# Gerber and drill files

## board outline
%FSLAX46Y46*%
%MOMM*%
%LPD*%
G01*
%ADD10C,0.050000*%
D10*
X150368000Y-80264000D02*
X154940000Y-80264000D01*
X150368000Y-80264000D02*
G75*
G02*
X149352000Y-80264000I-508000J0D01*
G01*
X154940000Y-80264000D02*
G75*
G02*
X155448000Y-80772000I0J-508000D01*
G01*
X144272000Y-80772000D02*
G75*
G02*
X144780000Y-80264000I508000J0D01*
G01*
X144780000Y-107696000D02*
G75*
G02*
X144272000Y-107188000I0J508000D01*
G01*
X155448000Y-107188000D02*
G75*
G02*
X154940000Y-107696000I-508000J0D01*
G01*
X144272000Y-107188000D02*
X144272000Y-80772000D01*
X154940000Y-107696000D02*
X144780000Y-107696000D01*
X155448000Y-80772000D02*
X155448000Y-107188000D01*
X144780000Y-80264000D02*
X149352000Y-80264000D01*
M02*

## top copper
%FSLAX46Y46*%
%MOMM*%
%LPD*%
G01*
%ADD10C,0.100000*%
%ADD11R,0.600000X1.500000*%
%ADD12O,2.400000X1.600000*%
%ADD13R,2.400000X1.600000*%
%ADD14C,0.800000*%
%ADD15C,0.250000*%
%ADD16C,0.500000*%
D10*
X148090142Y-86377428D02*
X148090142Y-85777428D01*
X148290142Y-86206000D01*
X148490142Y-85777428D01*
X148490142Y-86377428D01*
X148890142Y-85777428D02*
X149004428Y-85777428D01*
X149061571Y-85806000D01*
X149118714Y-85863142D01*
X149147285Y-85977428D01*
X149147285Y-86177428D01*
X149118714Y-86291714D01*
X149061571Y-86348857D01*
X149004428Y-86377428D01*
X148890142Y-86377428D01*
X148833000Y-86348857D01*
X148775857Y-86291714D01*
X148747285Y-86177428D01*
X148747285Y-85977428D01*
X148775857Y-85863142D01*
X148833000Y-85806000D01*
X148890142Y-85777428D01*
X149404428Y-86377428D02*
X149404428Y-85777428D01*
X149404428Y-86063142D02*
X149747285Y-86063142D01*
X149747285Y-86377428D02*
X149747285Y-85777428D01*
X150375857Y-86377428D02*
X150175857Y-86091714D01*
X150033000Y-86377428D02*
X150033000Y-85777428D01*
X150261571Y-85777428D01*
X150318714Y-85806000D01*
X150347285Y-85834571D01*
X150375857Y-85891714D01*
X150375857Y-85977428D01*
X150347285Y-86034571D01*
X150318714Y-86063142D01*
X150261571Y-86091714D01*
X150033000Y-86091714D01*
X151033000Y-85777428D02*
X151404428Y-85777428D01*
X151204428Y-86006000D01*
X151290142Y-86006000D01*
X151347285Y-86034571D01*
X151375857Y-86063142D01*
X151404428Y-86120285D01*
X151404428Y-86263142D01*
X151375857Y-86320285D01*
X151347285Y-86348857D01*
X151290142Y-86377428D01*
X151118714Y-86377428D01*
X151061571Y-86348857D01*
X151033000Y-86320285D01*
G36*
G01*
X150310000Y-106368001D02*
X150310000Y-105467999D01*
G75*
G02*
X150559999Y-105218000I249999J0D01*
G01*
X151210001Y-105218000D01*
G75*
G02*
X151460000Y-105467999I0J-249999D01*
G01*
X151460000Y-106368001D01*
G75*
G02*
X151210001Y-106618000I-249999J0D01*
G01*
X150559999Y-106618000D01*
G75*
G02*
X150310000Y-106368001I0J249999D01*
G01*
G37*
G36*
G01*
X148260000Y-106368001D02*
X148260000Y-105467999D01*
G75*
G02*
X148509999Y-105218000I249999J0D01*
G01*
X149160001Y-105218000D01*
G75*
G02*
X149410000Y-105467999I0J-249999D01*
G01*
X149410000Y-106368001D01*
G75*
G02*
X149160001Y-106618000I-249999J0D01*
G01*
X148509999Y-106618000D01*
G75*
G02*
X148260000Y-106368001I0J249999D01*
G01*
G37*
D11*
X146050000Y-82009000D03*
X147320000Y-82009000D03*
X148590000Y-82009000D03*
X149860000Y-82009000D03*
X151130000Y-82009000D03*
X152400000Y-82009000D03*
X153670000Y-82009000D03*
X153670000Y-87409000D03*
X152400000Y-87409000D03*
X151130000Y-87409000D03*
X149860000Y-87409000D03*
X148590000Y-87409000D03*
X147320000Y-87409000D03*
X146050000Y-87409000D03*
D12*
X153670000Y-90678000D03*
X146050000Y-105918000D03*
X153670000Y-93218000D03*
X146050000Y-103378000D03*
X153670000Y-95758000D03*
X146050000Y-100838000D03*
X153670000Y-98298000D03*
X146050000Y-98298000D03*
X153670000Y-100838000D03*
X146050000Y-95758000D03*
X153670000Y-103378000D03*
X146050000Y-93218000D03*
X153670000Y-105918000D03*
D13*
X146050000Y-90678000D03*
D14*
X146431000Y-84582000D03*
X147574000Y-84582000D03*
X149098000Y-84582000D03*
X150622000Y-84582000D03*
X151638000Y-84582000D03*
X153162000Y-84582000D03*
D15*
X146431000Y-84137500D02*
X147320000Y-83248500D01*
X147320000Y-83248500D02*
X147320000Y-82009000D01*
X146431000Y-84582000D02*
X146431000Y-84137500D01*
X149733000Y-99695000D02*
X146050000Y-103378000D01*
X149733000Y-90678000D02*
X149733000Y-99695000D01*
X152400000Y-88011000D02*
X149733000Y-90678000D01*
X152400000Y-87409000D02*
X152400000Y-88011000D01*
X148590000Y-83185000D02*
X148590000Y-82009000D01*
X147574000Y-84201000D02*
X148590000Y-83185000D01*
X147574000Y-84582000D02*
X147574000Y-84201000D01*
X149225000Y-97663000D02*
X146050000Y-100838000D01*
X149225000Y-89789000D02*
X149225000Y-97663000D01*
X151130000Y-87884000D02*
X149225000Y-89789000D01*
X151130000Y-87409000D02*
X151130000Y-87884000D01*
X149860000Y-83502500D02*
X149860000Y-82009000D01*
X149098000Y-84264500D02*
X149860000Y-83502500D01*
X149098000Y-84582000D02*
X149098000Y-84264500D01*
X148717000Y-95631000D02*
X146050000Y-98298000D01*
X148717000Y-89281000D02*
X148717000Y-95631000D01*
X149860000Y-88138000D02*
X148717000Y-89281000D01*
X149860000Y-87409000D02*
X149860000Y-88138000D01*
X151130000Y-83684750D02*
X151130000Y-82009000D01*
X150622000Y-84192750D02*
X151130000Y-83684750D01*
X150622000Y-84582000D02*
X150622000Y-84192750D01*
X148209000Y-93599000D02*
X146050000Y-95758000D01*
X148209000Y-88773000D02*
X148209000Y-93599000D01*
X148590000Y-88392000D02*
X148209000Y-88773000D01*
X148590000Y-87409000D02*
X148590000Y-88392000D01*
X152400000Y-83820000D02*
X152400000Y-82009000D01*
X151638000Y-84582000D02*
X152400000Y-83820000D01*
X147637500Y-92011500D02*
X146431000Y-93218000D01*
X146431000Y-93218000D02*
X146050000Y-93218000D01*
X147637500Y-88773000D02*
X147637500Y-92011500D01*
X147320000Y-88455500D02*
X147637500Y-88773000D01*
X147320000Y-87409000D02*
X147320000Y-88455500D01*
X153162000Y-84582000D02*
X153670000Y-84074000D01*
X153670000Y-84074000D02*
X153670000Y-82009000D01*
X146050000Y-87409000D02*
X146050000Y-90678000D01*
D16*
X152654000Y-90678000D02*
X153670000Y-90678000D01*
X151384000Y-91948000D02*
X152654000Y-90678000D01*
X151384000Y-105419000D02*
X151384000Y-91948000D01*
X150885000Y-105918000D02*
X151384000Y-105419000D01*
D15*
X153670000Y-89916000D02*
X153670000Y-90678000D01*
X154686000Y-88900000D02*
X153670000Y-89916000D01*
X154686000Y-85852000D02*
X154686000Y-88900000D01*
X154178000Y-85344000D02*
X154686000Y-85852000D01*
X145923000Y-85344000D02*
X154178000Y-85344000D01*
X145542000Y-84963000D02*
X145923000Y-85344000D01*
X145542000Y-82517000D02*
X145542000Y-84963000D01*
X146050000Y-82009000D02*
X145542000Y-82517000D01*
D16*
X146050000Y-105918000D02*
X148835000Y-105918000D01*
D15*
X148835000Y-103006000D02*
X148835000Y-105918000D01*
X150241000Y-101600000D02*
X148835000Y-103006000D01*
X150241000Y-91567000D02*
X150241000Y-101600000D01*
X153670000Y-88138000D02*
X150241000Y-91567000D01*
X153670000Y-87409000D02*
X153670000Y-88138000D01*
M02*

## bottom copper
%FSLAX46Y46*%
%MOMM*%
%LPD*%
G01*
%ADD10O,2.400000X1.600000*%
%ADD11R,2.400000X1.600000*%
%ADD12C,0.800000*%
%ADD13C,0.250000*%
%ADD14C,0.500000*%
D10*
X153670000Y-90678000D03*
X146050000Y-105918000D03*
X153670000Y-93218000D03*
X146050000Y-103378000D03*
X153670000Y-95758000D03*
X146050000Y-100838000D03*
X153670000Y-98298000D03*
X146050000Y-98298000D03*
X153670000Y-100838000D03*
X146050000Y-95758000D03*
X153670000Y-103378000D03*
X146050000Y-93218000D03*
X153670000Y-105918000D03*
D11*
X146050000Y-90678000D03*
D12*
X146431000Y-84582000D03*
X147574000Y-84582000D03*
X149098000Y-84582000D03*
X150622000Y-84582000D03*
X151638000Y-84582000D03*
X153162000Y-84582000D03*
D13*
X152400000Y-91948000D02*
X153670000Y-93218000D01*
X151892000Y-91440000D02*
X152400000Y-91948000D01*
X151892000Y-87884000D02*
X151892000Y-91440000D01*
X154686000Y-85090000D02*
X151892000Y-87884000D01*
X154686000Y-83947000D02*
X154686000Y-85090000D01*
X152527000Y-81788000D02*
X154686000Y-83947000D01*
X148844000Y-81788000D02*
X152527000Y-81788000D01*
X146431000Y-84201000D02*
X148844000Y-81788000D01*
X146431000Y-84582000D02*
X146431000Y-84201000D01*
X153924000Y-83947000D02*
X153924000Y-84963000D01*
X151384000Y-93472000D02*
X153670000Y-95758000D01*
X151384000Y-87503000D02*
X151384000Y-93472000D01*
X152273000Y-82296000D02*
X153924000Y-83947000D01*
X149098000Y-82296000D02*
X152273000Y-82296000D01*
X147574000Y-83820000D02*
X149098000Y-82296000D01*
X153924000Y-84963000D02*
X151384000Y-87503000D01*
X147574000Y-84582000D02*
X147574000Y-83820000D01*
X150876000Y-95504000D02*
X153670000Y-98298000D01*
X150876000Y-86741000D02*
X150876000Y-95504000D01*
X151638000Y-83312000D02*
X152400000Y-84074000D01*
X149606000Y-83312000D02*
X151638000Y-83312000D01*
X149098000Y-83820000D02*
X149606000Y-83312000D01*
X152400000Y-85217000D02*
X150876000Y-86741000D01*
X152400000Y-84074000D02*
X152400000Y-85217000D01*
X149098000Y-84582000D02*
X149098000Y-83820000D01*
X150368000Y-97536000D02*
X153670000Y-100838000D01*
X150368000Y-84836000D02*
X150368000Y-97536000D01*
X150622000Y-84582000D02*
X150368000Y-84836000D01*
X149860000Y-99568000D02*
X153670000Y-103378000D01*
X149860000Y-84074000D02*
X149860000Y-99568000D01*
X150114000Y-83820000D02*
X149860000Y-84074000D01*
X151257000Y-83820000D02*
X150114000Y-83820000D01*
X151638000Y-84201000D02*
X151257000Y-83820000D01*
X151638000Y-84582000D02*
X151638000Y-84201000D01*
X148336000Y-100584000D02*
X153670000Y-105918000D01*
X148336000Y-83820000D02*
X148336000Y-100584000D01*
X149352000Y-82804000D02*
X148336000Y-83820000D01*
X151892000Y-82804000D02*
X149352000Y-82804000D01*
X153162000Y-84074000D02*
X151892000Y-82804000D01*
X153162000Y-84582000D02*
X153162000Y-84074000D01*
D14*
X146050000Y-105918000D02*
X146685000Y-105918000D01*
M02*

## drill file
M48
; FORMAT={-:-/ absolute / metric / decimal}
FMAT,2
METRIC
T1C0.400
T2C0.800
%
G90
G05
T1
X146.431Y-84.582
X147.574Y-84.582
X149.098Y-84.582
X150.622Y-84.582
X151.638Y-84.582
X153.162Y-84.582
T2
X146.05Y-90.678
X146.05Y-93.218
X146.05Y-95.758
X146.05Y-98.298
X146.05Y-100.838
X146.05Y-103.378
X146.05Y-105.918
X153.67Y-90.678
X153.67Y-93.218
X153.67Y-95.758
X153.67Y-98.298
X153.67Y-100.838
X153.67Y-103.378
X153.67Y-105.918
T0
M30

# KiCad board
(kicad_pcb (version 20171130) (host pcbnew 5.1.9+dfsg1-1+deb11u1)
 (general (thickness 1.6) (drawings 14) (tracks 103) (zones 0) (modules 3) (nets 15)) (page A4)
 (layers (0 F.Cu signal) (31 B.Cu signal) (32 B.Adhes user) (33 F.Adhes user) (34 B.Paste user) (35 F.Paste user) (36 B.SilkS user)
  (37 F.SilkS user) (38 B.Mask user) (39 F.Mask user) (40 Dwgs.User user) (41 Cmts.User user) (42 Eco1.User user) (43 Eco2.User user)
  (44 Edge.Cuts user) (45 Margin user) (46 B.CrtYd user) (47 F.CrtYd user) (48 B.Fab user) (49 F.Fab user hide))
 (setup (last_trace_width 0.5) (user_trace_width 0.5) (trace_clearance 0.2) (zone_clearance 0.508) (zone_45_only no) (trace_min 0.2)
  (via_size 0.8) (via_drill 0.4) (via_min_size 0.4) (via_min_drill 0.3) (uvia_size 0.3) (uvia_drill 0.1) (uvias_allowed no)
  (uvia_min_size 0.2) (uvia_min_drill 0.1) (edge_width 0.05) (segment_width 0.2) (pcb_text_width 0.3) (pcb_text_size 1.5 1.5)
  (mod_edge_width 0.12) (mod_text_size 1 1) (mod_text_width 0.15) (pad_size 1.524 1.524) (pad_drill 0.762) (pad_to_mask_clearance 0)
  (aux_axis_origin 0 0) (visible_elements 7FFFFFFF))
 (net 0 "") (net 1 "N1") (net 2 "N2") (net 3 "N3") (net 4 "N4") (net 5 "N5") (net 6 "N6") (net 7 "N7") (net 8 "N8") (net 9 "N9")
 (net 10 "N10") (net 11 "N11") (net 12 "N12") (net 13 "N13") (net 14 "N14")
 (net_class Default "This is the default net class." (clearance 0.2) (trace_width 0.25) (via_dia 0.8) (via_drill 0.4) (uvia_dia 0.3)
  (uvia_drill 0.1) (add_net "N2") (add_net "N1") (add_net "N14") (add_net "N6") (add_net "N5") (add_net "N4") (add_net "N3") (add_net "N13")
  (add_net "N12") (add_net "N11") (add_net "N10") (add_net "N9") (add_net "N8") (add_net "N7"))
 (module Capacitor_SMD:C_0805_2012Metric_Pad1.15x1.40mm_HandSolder (layer F.Cu) (at 149.86 105.918)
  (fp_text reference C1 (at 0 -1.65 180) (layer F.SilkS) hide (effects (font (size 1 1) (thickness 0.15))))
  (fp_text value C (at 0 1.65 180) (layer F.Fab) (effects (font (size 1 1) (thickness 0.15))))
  (pad 2 smd roundrect (at 1.025 0) (size 1.15 1.4) (layers F.Cu F.Paste F.Mask) (roundrect_rratio 0.217391) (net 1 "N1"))
  (pad 1 smd roundrect (at -1.025 0) (size 1.15 1.4) (layers F.Cu F.Paste F.Mask) (roundrect_rratio 0.217391) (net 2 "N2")))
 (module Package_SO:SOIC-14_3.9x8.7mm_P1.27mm (layer F.Cu) (at 149.86 84.709 90)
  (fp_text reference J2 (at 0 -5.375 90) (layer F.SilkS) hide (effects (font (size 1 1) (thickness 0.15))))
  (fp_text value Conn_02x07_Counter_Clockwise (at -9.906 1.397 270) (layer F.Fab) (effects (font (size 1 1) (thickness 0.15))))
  (pad 14 smd rect (at 2.7 -3.81 90) (size 1.5 0.6) (layers F.Cu F.Paste F.Mask) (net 1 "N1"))
  (pad 13 smd rect (at 2.7 -2.54 90) (size 1.5 0.6) (layers F.Cu F.Paste F.Mask) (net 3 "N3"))
  (pad 12 smd rect (at 2.7 -1.27 90) (size 1.5 0.6) (layers F.Cu F.Paste F.Mask) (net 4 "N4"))
  (pad 11 smd rect (at 2.7 0 90) (size 1.5 0.6) (layers F.Cu F.Paste F.Mask) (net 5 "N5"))
  (pad 10 smd rect (at 2.7 1.27 90) (size 1.5 0.6) (layers F.Cu F.Paste F.Mask) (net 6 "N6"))
  (pad 9 smd rect (at 2.7 2.54 90) (size 1.5 0.6) (layers F.Cu F.Paste F.Mask) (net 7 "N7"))
  (pad 8 smd rect (at 2.7 3.81 90) (size 1.5 0.6) (layers F.Cu F.Paste F.Mask) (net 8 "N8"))
  (pad 7 smd rect (at -2.7 3.81 90) (size 1.5 0.6) (layers F.Cu F.Paste F.Mask) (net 2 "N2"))
  (pad 6 smd rect (at -2.7 2.54 90) (size 1.5 0.6) (layers F.Cu F.Paste F.Mask) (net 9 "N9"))
  (pad 5 smd rect (at -2.7 1.27 90) (size 1.5 0.6) (layers F.Cu F.Paste F.Mask) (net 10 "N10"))
  (pad 4 smd rect (at -2.7 0 90) (size 1.5 0.6) (layers F.Cu F.Paste F.Mask) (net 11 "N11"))
  (pad 3 smd rect (at -2.7 -1.27 90) (size 1.5 0.6) (layers F.Cu F.Paste F.Mask) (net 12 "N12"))
  (pad 2 smd rect (at -2.7 -2.54 90) (size 1.5 0.6) (layers F.Cu F.Paste F.Mask) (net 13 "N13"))
  (pad 1 smd rect (at -2.7 -3.81 90) (size 1.5 0.6) (layers F.Cu F.Paste F.Mask) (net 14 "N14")))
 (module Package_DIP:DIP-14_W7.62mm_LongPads (layer F.Cu) (at 146.05 90.678)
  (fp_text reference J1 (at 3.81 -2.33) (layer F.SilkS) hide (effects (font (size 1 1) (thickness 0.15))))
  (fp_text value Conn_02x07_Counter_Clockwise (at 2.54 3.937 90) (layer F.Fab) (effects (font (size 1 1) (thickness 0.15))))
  (pad 14 thru_hole oval (at 7.62 0) (size 2.4 1.6) (drill 0.8) (layers *.Cu *.Mask) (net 1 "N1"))
  (pad 7 thru_hole oval (at 0 15.24) (size 2.4 1.6) (drill 0.8) (layers *.Cu *.Mask) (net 2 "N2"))
  (pad 13 thru_hole oval (at 7.62 2.54) (size 2.4 1.6) (drill 0.8) (layers *.Cu *.Mask) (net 3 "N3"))
  (pad 6 thru_hole oval (at 0 12.7) (size 2.4 1.6) (drill 0.8) (layers *.Cu *.Mask) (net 9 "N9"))
  (pad 12 thru_hole oval (at 7.62 5.08) (size 2.4 1.6) (drill 0.8) (layers *.Cu *.Mask) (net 4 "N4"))
  (pad 5 thru_hole oval (at 0 10.16) (size 2.4 1.6) (drill 0.8) (layers *.Cu *.Mask) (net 10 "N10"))
  (pad 11 thru_hole oval (at 7.62 7.62) (size 2.4 1.6) (drill 0.8) (layers *.Cu *.Mask) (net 5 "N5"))
  (pad 4 thru_hole oval (at 0 7.62) (size 2.4 1.6) (drill 0.8) (layers *.Cu *.Mask) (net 11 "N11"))
  (pad 10 thru_hole oval (at 7.62 10.16) (size 2.4 1.6) (drill 0.8) (layers *.Cu *.Mask) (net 6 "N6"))
  (pad 3 thru_hole oval (at 0 5.08) (size 2.4 1.6) (drill 0.8) (layers *.Cu *.Mask) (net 12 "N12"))
  (pad 9 thru_hole oval (at 7.62 12.7) (size 2.4 1.6) (drill 0.8) (layers *.Cu *.Mask) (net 7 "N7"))
  (pad 2 thru_hole oval (at 0 2.54) (size 2.4 1.6) (drill 0.8) (layers *.Cu *.Mask) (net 13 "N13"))
  (pad 8 thru_hole oval (at 7.62 15.24) (size 2.4 1.6) (drill 0.8) (layers *.Cu *.Mask) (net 8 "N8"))
  (pad 1 thru_hole rect (at 0 0) (size 2.4 1.6) (drill 0.8) (layers *.Cu *.Mask) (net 14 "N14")))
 (gr_line (start 150.368 80.264) (end 154.94 80.264) (layer Edge.Cuts) (width 0.05))
 (gr_arc (start 149.86 80.264) (end 149.352 80.264) (angle -180) (layer Edge.Cuts) (width 0.05))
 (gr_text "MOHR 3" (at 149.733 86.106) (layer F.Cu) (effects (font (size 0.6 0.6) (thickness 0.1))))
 (gr_arc (start 154.94 80.772) (end 155.448 80.772) (angle -90) (layer Edge.Cuts) (width 0.05))
 (gr_arc (start 144.78 80.772) (end 144.78 80.264) (angle -90) (layer Edge.Cuts) (width 0.05))
 (gr_arc (start 144.78 107.188) (end 144.272 107.188) (angle -90) (layer Edge.Cuts) (width 0.05))
 (gr_arc (start 154.94 107.188) (end 154.94 107.696) (angle -90) (layer Edge.Cuts) (width 0.05))
 (gr_line (start 144.272 107.188) (end 144.272 80.772) (layer Edge.Cuts) (width 0.05))
 (gr_line (start 154.94 107.696) (end 144.78 107.696) (layer Edge.Cuts) (width 0.05))
 (gr_line (start 155.448 80.772) (end 155.448 107.188) (layer Edge.Cuts) (width 0.05))
 (gr_line (start 144.78 80.264) (end 149.352 80.264) (layer Edge.Cuts) (width 0.05))
 (via (at 146.431 84.582) (size 0.8) (drill 0.4) (layers F.Cu B.Cu) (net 3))
 (segment (start 146.431 84.1375) (end 147.32 83.2485) (width 0.25) (layer F.Cu) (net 3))
 (segment (start 147.32 83.2485) (end 147.32 82.009) (width 0.25) (layer F.Cu) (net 3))
 (segment (start 146.431 84.582) (end 146.431 84.1375) (width 0.25) (layer F.Cu) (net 3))
 (segment (start 152.4 91.948) (end 153.67 93.218) (width 0.25) (layer B.Cu) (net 3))
 (segment (start 151.892 91.44) (end 152.4 91.948) (width 0.25) (layer B.Cu) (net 3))
 (segment (start 151.892 87.884) (end 151.892 91.44) (width 0.25) (layer B.Cu) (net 3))
 (segment (start 154.686 85.09) (end 151.892 87.884) (width 0.25) (layer B.Cu) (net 3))
 (segment (start 154.686 83.947) (end 154.686 85.09) (width 0.25) (layer B.Cu) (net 3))
 (segment (start 152.527 81.788) (end 154.686 83.947) (width 0.25) (layer B.Cu) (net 3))
 (segment (start 148.844 81.788) (end 152.527 81.788) (width 0.25) (layer B.Cu) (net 3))
 (segment (start 146.431 84.201) (end 148.844 81.788) (width 0.25) (layer B.Cu) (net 3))
 (segment (start 146.431 84.582) (end 146.431 84.201) (width 0.25) (layer B.Cu) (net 3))
 (segment (start 149.733 99.695) (end 146.05 103.378) (width 0.25) (layer F.Cu) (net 9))
 (segment (start 149.733 90.678) (end 149.733 99.695) (width 0.25) (layer F.Cu) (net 9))
 (segment (start 152.4 88.011) (end 149.733 90.678) (width 0.25) (layer F.Cu) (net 9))
 (segment (start 152.4 87.409) (end 152.4 88.011) (width 0.25) (layer F.Cu) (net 9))
 (via (at 147.574 84.582) (size 0.8) (drill 0.4) (layers F.Cu B.Cu) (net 4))
 (segment (start 148.59 83.185) (end 148.59 82.009) (width 0.25) (layer F.Cu) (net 4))
 (segment (start 147.574 84.201) (end 148.59 83.185) (width 0.25) (layer F.Cu) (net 4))
 (segment (start 147.574 84.582) (end 147.574 84.201) (width 0.25) (layer F.Cu) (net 4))
 (segment (start 153.924 83.947) (end 153.924 84.963) (width 0.25) (layer B.Cu) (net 4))
 (segment (start 151.384 93.472) (end 153.67 95.758) (width 0.25) (layer B.Cu) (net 4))
 (segment (start 151.384 87.503) (end 151.384 93.472) (width 0.25) (layer B.Cu) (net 4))
 (segment (start 152.273 82.296) (end 153.924 83.947) (width 0.25) (layer B.Cu) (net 4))
 (segment (start 149.098 82.296) (end 152.273 82.296) (width 0.25) (layer B.Cu) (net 4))
 (segment (start 147.574 83.82) (end 149.098 82.296) (width 0.25) (layer B.Cu) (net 4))
 (segment (start 153.924 84.963) (end 151.384 87.503) (width 0.25) (layer B.Cu) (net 4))
 (segment (start 147.574 84.582) (end 147.574 83.82) (width 0.25) (layer B.Cu) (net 4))
 (segment (start 149.225 97.663) (end 146.05 100.838) (width 0.25) (layer F.Cu) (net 10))
 (segment (start 149.225 89.789) (end 149.225 97.663) (width 0.25) (layer F.Cu) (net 10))
 (segment (start 151.13 87.884) (end 149.225 89.789) (width 0.25) (layer F.Cu) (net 10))
 (segment (start 151.13 87.409) (end 151.13 87.884) (width 0.25) (layer F.Cu) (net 10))
 (via (at 149.098 84.582) (size 0.8) (drill 0.4) (layers F.Cu B.Cu) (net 5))
 (segment (start 149.86 83.5025) (end 149.86 82.009) (width 0.25) (layer F.Cu) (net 5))
 (segment (start 149.098 84.2645) (end 149.86 83.5025) (width 0.25) (layer F.Cu) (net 5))
 (segment (start 149.098 84.582) (end 149.098 84.2645) (width 0.25) (layer F.Cu) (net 5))
 (segment (start 150.876 95.504) (end 153.67 98.298) (width 0.25) (layer B.Cu) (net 5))
 (segment (start 150.876 86.741) (end 150.876 95.504) (width 0.25) (layer B.Cu) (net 5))
 (segment (start 151.638 83.312) (end 152.4 84.074) (width 0.25) (layer B.Cu) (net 5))
 (segment (start 149.606 83.312) (end 151.638 83.312) (width 0.25) (layer B.Cu) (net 5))
 (segment (start 149.098 83.82) (end 149.606 83.312) (width 0.25) (layer B.Cu) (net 5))
 (segment (start 152.4 85.217) (end 150.876 86.741) (width 0.25) (layer B.Cu) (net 5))
 (segment (start 152.4 84.074) (end 152.4 85.217) (width 0.25) (layer B.Cu) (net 5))
 (segment (start 149.098 84.582) (end 149.098 83.82) (width 0.25) (layer B.Cu) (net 5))
 (segment (start 148.717 95.631) (end 146.05 98.298) (width 0.25) (layer F.Cu) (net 11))
 (segment (start 148.717 89.281) (end 148.717 95.631) (width 0.25) (layer F.Cu) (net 11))
 (segment (start 149.86 88.138) (end 148.717 89.281) (width 0.25) (layer F.Cu) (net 11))
 (segment (start 149.86 87.409) (end 149.86 88.138) (width 0.25) (layer F.Cu) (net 11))
 (via (at 150.622 84.582) (size 0.8) (drill 0.4) (layers F.Cu B.Cu) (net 6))
 (segment (start 151.13 83.68475) (end 151.13 82.009) (width 0.25) (layer F.Cu) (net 6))
 (segment (start 150.622 84.19275) (end 151.13 83.68475) (width 0.25) (layer F.Cu) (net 6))
 (segment (start 150.622 84.582) (end 150.622 84.19275) (width 0.25) (layer F.Cu) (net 6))
 (segment (start 150.368 97.536) (end 153.67 100.838) (width 0.25) (layer B.Cu) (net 6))
 (segment (start 150.368 84.836) (end 150.368 97.536) (width 0.25) (layer B.Cu) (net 6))
 (segment (start 150.622 84.582) (end 150.368 84.836) (width 0.25) (layer B.Cu) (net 6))
 (segment (start 148.209 93.599) (end 146.05 95.758) (width 0.25) (layer F.Cu) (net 12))
 (segment (start 148.209 88.773) (end 148.209 93.599) (width 0.25) (layer F.Cu) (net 12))
 (segment (start 148.59 88.392) (end 148.209 88.773) (width 0.25) (layer F.Cu) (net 12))
 (segment (start 148.59 87.409) (end 148.59 88.392) (width 0.25) (layer F.Cu) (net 12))
 (segment (start 152.4 83.82) (end 152.4 82.009) (width 0.25) (layer F.Cu) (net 7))
 (segment (start 151.638 84.582) (end 152.4 83.82) (width 0.25) (layer F.Cu) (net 7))
 (via (at 151.638 84.582) (size 0.8) (drill 0.4) (layers F.Cu B.Cu) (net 7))
 (segment (start 149.86 99.568) (end 153.67 103.378) (width 0.25) (layer B.Cu) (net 7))
 (segment (start 149.86 84.074) (end 149.86 99.568) (width 0.25) (layer B.Cu) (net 7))
 (segment (start 150.114 83.82) (end 149.86 84.074) (width 0.25) (layer B.Cu) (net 7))
 (segment (start 151.257 83.82) (end 150.114 83.82) (width 0.25) (layer B.Cu) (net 7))
 (segment (start 151.638 84.201) (end 151.257 83.82) (width 0.25) (layer B.Cu) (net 7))
 (segment (start 151.638 84.582) (end 151.638 84.201) (width 0.25) (layer B.Cu) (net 7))
 (segment (start 147.6375 92.0115) (end 146.431 93.218) (width 0.25) (layer F.Cu) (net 13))
 (segment (start 146.431 93.218) (end 146.05 93.218) (width 0.25) (layer F.Cu) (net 13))
 (segment (start 147.6375 88.773) (end 147.6375 92.0115) (width 0.25) (layer F.Cu) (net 13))
 (segment (start 147.32 88.4555) (end 147.6375 88.773) (width 0.25) (layer F.Cu) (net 13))
 (segment (start 147.32 87.409) (end 147.32 88.4555) (width 0.25) (layer F.Cu) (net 13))
 (segment (start 153.162 84.582) (end 153.67 84.074) (width 0.25) (layer F.Cu) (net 8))
 (segment (start 153.67 84.074) (end 153.67 82.009) (width 0.25) (layer F.Cu) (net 8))
 (via (at 153.162 84.582) (size 0.8) (drill 0.4) (layers F.Cu B.Cu) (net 8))
 (segment (start 148.336 100.584) (end 153.67 105.918) (width 0.25) (layer B.Cu) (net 8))
 (segment (start 148.336 83.82) (end 148.336 100.584) (width 0.25) (layer B.Cu) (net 8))
 (segment (start 149.352 82.804) (end 148.336 83.82) (width 0.25) (layer B.Cu) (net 8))
 (segment (start 151.892 82.804) (end 149.352 82.804) (width 0.25) (layer B.Cu) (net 8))
 (segment (start 153.162 84.074) (end 151.892 82.804) (width 0.25) (layer B.Cu) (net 8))
 (segment (start 153.162 84.582) (end 153.162 84.074) (width 0.25) (layer B.Cu) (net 8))
 (segment (start 146.05 87.409) (end 146.05 90.678) (width 0.25) (layer F.Cu) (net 14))
 (segment (start 152.654 90.678) (end 153.67 90.678) (width 0.5) (layer F.Cu) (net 1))
 (segment (start 151.384 91.948) (end 152.654 90.678) (width 0.5) (layer F.Cu) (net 1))
 (segment (start 151.384 105.419) (end 151.384 91.948) (width 0.5) (layer F.Cu) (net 1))
 (segment (start 150.885 105.918) (end 151.384 105.419) (width 0.5) (layer F.Cu) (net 1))
 (segment (start 153.67 89.916) (end 153.67 90.678) (width 0.25) (layer F.Cu) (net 1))
 (segment (start 154.686 88.9) (end 153.67 89.916) (width 0.25) (layer F.Cu) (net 1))
 (segment (start 154.686 85.852) (end 154.686 88.9) (width 0.25) (layer F.Cu) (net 1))
 (segment (start 154.178 85.344) (end 154.686 85.852) (width 0.25) (layer F.Cu) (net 1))
 (segment (start 145.923 85.344) (end 154.178 85.344) (width 0.25) (layer F.Cu) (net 1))
 (segment (start 145.542 84.963) (end 145.923 85.344) (width 0.25) (layer F.Cu) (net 1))
 (segment (start 145.542 82.517) (end 145.542 84.963) (width 0.25) (layer F.Cu) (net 1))
 (segment (start 146.05 82.009) (end 145.542 82.517) (width 0.25) (layer F.Cu) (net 1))
 (segment (start 146.05 105.918) (end 146.685 105.918) (width 0.5) (layer B.Cu) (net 2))
 (segment (start 146.05 105.918) (end 148.835 105.918) (width 0.5) (layer F.Cu) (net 2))
 (segment (start 148.835 103.006) (end 148.835 105.918) (width 0.25) (layer F.Cu) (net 2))
 (segment (start 150.241 101.6) (end 148.835 103.006) (width 0.25) (layer F.Cu) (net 2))
 (segment (start 150.241 91.567) (end 150.241 101.6) (width 0.25) (layer F.Cu) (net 2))
 (segment (start 153.67 88.138) (end 150.241 91.567) (width 0.25) (layer F.Cu) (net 2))
 (segment (start 153.67 87.409) (end 153.67 88.138) (width 0.25) (layer F.Cu) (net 2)))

